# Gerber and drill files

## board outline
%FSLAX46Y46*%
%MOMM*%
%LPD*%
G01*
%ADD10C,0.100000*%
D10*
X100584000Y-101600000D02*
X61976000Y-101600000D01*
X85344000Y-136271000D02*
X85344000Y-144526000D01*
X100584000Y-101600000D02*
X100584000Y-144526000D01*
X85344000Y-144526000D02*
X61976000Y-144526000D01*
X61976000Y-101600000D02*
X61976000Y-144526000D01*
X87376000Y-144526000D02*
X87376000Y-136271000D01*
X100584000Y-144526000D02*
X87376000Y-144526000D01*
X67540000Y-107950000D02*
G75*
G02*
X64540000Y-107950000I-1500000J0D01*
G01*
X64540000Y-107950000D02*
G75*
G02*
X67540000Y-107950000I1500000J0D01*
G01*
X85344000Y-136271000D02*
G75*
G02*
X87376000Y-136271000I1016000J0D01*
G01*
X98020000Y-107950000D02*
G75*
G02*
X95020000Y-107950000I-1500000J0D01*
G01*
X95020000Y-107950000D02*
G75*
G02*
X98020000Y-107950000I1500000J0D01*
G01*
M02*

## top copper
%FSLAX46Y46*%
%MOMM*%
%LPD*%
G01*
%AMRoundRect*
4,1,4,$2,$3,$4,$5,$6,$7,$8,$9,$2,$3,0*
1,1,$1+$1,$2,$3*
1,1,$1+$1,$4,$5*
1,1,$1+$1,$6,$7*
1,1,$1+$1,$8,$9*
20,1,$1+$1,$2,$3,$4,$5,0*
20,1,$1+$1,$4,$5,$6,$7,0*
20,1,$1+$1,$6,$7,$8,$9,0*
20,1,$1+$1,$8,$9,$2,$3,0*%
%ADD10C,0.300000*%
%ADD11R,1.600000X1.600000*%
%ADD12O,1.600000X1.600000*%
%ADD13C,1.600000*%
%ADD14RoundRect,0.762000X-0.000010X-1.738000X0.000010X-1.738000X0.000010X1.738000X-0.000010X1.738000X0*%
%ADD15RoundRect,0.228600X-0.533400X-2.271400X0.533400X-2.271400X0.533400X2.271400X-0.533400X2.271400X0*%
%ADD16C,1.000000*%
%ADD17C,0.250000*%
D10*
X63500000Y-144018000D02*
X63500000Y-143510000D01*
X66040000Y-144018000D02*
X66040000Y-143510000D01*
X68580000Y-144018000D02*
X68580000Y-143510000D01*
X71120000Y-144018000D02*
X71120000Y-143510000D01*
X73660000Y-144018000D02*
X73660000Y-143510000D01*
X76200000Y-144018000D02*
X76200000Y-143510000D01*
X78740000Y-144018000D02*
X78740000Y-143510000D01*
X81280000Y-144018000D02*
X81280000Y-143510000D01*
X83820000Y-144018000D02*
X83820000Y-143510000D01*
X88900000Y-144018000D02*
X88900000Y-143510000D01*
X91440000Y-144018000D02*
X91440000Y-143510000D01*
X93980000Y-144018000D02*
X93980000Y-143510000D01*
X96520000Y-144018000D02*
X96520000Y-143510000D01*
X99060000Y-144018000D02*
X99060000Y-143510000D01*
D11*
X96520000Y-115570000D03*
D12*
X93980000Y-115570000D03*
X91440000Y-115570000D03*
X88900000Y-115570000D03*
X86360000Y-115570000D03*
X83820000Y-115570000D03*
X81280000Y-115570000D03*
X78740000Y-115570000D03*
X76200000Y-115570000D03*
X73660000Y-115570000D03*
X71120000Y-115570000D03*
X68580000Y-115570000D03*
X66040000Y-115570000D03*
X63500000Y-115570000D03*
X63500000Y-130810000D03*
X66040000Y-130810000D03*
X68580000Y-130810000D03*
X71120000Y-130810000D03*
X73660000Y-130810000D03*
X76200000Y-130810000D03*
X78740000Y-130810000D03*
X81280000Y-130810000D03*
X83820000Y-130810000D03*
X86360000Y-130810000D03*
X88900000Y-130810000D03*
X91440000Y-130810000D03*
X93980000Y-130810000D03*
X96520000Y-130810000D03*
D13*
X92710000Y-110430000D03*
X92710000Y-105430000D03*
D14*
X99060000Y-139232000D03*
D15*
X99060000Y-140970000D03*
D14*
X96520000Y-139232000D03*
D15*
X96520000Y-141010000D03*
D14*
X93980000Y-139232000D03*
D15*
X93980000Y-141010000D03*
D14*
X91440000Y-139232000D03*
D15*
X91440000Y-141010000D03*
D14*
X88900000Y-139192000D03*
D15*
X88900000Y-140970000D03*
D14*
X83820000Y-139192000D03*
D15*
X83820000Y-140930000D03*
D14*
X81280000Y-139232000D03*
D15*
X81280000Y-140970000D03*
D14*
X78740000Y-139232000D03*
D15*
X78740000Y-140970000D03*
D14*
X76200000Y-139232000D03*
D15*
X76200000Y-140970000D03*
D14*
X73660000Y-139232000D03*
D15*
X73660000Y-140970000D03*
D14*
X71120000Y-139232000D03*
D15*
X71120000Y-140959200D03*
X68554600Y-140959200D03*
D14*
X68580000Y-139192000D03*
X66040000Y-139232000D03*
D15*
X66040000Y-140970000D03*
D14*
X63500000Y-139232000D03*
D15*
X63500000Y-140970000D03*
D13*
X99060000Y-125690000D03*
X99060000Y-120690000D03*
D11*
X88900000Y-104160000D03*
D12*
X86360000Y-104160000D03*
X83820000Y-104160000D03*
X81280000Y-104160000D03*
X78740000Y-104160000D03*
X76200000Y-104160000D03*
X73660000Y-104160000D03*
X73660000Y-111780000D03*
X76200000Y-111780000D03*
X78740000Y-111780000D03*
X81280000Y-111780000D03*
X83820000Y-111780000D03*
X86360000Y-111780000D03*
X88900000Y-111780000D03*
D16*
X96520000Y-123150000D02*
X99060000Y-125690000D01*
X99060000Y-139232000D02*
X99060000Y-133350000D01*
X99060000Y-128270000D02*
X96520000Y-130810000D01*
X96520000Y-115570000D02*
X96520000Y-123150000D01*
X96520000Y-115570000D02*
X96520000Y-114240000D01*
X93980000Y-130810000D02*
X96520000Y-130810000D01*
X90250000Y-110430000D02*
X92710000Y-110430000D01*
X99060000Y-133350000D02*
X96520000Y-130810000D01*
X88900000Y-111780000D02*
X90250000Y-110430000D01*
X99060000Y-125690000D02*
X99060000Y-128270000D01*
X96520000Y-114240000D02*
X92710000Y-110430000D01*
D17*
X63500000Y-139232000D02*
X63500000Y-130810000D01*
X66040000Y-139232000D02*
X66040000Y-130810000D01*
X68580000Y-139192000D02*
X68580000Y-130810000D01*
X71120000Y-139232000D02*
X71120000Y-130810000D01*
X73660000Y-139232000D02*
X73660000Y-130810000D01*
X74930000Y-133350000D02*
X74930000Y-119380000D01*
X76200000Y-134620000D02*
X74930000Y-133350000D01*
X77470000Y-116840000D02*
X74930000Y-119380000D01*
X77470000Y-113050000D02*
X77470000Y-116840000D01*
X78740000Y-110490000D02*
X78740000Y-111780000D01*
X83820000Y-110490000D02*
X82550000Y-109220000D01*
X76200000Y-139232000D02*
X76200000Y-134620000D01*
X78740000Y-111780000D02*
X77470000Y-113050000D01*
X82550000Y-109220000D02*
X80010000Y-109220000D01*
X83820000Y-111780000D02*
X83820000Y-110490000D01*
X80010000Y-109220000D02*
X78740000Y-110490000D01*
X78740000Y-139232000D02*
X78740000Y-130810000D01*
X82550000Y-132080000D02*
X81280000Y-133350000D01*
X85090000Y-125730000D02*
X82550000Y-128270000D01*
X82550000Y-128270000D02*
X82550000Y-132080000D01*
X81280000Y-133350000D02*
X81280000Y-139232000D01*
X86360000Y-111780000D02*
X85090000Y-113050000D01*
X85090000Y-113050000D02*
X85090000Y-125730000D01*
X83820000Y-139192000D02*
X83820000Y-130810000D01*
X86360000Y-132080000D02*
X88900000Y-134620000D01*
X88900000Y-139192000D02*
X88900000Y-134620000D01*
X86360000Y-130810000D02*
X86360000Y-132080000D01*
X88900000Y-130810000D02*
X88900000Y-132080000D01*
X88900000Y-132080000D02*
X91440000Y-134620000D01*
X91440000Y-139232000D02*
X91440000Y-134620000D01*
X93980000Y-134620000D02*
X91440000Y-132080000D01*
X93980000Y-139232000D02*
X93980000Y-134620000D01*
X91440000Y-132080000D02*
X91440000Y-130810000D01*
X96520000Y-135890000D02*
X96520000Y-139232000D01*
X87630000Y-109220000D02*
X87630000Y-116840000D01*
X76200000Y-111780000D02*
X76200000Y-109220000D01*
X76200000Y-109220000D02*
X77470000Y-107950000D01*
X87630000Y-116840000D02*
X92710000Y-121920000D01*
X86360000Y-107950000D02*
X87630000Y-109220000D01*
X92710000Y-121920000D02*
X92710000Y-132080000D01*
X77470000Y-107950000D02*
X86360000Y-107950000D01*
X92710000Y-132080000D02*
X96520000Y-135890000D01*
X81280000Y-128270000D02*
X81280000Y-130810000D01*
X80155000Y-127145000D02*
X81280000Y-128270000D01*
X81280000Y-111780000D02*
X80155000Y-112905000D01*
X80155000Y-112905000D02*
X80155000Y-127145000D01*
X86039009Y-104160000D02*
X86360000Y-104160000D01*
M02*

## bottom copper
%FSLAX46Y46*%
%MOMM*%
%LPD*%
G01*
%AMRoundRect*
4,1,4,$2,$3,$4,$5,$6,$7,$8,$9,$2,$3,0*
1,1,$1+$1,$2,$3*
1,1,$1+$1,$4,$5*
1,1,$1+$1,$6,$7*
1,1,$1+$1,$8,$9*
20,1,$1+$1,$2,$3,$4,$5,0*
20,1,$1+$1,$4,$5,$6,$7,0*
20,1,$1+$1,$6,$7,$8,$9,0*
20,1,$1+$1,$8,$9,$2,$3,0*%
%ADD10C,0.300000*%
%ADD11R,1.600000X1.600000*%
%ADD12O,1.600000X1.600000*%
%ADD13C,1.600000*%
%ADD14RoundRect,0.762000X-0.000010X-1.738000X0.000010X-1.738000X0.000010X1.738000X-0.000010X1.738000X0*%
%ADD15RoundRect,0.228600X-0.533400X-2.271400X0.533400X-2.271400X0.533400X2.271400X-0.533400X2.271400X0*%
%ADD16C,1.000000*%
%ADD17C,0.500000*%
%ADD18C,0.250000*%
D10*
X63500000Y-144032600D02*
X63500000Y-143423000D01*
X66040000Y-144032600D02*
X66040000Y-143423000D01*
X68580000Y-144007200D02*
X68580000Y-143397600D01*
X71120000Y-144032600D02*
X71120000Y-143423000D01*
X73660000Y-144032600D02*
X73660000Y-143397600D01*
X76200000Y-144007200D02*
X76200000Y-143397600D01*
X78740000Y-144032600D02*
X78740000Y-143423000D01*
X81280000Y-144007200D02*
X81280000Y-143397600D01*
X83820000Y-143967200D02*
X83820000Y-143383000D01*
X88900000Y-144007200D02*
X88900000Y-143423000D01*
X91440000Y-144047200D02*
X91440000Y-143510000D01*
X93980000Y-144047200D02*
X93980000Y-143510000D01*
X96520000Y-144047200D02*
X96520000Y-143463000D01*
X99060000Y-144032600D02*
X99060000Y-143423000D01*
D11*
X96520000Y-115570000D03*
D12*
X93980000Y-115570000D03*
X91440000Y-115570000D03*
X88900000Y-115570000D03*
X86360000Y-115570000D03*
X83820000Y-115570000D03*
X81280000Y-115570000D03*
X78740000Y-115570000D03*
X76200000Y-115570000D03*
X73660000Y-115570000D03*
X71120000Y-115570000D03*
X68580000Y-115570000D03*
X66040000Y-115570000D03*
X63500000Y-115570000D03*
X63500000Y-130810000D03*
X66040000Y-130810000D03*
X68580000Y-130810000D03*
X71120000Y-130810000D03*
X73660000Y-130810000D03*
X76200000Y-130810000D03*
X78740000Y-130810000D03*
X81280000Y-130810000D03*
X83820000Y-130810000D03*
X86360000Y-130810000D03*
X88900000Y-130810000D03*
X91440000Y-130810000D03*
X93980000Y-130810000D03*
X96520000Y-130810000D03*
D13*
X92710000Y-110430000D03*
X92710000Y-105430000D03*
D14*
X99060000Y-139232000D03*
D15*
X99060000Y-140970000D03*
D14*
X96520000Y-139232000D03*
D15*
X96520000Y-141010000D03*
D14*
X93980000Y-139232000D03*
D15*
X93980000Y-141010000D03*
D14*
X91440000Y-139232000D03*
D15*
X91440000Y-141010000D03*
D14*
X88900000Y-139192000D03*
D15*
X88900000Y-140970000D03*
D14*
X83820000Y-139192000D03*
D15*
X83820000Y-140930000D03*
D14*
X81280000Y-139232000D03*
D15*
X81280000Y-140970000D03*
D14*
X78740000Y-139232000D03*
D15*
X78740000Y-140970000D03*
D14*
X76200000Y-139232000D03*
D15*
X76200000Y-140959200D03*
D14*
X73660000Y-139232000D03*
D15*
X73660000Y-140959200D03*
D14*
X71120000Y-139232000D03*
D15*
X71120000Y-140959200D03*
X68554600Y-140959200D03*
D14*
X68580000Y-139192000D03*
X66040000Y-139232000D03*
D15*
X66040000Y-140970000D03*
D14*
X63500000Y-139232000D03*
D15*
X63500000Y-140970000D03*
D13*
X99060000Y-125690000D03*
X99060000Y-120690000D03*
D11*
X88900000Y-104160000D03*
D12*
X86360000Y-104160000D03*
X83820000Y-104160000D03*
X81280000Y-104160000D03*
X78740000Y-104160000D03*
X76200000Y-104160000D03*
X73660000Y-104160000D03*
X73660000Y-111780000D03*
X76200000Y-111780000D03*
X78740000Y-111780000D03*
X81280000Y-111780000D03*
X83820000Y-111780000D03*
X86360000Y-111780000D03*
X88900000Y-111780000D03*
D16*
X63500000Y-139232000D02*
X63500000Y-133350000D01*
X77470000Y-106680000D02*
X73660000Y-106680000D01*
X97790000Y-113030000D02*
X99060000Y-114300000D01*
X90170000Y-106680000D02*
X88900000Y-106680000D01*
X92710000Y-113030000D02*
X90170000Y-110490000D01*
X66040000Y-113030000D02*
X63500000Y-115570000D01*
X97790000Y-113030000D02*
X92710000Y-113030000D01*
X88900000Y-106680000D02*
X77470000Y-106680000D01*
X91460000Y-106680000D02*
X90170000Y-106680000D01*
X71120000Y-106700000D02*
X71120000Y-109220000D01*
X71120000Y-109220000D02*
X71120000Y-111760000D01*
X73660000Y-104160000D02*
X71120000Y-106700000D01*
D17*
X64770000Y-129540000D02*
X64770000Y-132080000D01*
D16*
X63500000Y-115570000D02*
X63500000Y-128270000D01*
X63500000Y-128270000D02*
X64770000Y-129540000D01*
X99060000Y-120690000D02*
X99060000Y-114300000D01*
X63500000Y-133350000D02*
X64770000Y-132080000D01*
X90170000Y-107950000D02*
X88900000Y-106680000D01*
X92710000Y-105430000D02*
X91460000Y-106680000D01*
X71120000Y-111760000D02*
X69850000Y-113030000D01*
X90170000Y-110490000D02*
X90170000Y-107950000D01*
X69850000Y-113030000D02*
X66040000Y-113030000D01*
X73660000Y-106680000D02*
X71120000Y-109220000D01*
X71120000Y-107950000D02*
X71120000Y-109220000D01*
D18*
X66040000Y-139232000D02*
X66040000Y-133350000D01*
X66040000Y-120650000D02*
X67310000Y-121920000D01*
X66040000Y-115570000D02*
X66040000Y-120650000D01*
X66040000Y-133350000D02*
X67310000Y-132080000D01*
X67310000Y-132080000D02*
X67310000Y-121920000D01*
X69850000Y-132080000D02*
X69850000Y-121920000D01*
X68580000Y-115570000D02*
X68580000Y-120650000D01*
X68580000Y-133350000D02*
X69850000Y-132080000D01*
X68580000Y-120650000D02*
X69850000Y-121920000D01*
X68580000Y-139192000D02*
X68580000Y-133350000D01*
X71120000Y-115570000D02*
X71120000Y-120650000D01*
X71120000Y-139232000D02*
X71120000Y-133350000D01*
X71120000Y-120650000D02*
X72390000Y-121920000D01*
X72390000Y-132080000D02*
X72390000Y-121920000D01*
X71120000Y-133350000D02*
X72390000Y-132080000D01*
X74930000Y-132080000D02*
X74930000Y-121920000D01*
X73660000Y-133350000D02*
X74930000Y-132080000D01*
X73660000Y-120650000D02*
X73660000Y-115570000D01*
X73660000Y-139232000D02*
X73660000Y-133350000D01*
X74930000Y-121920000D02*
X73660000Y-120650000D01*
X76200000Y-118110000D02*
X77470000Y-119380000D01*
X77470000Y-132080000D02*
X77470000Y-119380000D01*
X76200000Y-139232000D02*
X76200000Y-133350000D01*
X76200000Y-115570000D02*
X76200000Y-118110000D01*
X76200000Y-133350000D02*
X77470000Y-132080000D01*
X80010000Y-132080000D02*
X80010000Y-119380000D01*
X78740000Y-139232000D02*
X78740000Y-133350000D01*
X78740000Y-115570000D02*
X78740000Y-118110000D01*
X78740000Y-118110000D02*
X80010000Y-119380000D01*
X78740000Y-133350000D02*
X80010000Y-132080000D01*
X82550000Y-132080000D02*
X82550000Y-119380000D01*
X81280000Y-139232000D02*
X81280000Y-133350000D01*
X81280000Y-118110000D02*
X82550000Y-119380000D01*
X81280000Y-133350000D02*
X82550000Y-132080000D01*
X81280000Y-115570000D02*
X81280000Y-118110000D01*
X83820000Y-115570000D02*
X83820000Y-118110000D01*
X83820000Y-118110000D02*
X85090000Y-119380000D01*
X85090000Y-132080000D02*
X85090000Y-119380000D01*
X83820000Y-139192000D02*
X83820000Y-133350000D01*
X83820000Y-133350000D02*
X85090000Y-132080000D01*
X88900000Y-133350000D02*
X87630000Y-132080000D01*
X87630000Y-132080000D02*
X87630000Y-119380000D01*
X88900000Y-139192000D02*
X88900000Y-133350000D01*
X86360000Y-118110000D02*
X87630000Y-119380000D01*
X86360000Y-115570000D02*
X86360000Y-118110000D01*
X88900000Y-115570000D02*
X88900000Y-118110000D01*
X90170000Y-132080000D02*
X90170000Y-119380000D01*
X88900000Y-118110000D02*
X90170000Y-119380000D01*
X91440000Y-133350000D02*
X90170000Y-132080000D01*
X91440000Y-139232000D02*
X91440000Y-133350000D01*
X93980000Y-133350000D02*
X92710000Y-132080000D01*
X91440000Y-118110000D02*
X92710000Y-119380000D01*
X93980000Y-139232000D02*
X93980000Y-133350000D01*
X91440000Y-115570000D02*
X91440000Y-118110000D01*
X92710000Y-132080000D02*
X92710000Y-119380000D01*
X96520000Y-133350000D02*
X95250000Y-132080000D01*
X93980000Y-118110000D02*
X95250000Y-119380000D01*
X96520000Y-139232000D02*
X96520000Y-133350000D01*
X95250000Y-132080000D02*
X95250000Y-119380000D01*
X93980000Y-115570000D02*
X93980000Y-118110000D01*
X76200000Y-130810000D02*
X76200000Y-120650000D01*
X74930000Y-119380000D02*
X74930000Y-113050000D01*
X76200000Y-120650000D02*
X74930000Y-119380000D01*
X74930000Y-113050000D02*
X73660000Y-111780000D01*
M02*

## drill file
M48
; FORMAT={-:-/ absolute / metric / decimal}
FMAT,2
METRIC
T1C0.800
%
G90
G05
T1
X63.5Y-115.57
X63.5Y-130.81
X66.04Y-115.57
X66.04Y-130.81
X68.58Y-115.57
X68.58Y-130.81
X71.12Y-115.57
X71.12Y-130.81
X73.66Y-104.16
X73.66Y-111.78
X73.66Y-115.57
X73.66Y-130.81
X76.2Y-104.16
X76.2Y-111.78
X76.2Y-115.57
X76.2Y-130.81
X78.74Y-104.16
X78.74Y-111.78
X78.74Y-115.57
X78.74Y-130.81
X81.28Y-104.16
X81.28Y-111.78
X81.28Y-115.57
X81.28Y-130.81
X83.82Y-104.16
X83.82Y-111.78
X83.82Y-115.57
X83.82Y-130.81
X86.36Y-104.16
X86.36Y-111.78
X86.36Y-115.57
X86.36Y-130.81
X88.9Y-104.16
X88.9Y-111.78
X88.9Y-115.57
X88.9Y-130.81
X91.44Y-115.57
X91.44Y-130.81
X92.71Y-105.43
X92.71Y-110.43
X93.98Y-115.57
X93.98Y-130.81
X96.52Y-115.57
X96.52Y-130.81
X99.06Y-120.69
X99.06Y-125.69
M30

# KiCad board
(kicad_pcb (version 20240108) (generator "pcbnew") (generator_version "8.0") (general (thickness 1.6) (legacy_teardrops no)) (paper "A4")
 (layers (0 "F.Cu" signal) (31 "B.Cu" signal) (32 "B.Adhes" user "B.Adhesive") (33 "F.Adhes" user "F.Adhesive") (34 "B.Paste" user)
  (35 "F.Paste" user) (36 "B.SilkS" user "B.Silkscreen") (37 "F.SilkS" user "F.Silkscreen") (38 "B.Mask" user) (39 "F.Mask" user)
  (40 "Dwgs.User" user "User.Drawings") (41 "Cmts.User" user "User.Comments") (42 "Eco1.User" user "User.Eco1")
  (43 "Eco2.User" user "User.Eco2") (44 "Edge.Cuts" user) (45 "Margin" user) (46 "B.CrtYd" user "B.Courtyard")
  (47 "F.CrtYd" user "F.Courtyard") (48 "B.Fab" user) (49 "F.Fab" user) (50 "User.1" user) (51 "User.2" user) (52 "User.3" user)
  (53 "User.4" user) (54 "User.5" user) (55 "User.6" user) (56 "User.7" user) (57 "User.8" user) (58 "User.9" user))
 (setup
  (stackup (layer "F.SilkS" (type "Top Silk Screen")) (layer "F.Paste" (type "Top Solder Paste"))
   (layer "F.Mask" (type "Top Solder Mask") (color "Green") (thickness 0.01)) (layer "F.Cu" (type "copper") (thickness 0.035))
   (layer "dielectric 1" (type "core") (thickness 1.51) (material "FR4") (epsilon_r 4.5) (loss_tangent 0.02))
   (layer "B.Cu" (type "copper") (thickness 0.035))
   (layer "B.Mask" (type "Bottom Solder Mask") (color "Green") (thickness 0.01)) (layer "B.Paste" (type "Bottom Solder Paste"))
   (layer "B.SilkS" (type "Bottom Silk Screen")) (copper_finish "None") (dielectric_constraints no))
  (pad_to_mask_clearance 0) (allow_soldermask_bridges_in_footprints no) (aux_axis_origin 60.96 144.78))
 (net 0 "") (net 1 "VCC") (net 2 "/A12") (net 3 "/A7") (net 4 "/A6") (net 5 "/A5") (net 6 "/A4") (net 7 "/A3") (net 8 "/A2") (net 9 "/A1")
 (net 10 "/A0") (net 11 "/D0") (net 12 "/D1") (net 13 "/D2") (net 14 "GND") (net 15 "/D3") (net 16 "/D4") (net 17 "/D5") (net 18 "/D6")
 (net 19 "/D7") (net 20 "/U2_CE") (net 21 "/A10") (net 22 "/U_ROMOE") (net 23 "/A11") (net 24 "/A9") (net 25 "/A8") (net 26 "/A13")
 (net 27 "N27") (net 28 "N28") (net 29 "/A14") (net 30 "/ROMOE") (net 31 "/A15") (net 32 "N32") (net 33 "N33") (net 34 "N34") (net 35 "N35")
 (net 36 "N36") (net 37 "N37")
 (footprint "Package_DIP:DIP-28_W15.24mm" (layer "F.Cu") (at 96.52 115.57 -90)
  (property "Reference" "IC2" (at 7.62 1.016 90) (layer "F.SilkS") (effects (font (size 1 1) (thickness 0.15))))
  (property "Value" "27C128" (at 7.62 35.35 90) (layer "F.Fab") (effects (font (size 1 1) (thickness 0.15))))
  (pad "1" thru_hole rect (at 0 0 270) (size 1.6 1.6) (drill 0.8) (layers "*.Cu" "*.Mask") (remove_unused_layers no) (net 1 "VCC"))
  (pad "2" thru_hole oval (at 0 2.54 270) (size 1.6 1.6) (drill 0.8) (layers "*.Cu" "*.Mask") (remove_unused_layers no) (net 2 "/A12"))
  (pad "3" thru_hole oval (at 0 5.08 270) (size 1.6 1.6) (drill 0.8) (layers "*.Cu" "*.Mask") (remove_unused_layers no) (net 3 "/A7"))
  (pad "4" thru_hole oval (at 0 7.62 270) (size 1.6 1.6) (drill 0.8) (layers "*.Cu" "*.Mask") (remove_unused_layers no) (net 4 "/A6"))
  (pad "5" thru_hole oval (at 0 10.16 270) (size 1.6 1.6) (drill 0.8) (layers "*.Cu" "*.Mask") (remove_unused_layers no) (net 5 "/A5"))
  (pad "6" thru_hole oval (at 0 12.7 270) (size 1.6 1.6) (drill 0.8) (layers "*.Cu" "*.Mask") (remove_unused_layers no) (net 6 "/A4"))
  (pad "7" thru_hole oval (at 0 15.24 270) (size 1.6 1.6) (drill 0.8) (layers "*.Cu" "*.Mask") (remove_unused_layers no) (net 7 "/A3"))
  (pad "8" thru_hole oval (at 0 17.78 270) (size 1.6 1.6) (drill 0.8) (layers "*.Cu" "*.Mask") (remove_unused_layers no) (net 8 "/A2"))
  (pad "9" thru_hole oval (at 0 20.32 270) (size 1.6 1.6) (drill 0.8) (layers "*.Cu" "*.Mask") (remove_unused_layers no) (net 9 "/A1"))
  (pad "10" thru_hole oval (at 0 22.86 270) (size 1.6 1.6) (drill 0.8) (layers "*.Cu" "*.Mask") (remove_unused_layers no) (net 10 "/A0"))
  (pad "11" thru_hole oval (at 0 25.4 270) (size 1.6 1.6) (drill 0.8) (layers "*.Cu" "*.Mask") (remove_unused_layers no) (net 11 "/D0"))
  (pad "12" thru_hole oval (at 0 27.94 270) (size 1.6 1.6) (drill 0.8) (layers "*.Cu" "*.Mask") (remove_unused_layers no) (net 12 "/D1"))
  (pad "13" thru_hole oval (at 0 30.48 270) (size 1.6 1.6) (drill 0.8) (layers "*.Cu" "*.Mask") (remove_unused_layers no) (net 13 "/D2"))
  (pad "14" thru_hole oval (at 0 33.02 270) (size 1.6 1.6) (drill 0.8) (layers "*.Cu" "*.Mask") (remove_unused_layers no) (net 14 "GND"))
  (pad "15" thru_hole oval (at 15.24 33.02 270) (size 1.6 1.6) (drill 0.8) (layers "*.Cu" "*.Mask") (remove_unused_layers no) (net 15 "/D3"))
  (pad "16" thru_hole oval (at 15.24 30.48 270) (size 1.6 1.6) (drill 0.8) (layers "*.Cu" "*.Mask") (remove_unused_layers no) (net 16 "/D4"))
  (pad "17" thru_hole oval (at 15.24 27.94 270) (size 1.6 1.6) (drill 0.8) (layers "*.Cu" "*.Mask") (remove_unused_layers no) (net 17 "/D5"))
  (pad "18" thru_hole oval (at 15.24 25.4 270) (size 1.6 1.6) (drill 0.8) (layers "*.Cu" "*.Mask") (remove_unused_layers no) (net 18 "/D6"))
  (pad "19" thru_hole oval (at 15.24 22.86 270) (size 1.6 1.6) (drill 0.8) (layers "*.Cu" "*.Mask") (remove_unused_layers no) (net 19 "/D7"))
  (pad "20" thru_hole oval (at 15.24 20.32 270) (size 1.6 1.6) (drill 0.8) (layers "*.Cu" "*.Mask") (remove_unused_layers no)
   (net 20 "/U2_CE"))
  (pad "21" thru_hole oval (at 15.24 17.78 270) (size 1.6 1.6) (drill 0.8) (layers "*.Cu" "*.Mask") (remove_unused_layers no)
   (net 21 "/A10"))
  (pad "22" thru_hole oval (at 15.24 15.24 270) (size 1.6 1.6) (drill 0.8) (layers "*.Cu" "*.Mask") (remove_unused_layers no)
   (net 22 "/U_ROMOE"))
  (pad "23" thru_hole oval (at 15.24 12.7 270) (size 1.6 1.6) (drill 0.8) (layers "*.Cu" "*.Mask") (remove_unused_layers no) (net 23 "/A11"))
  (pad "24" thru_hole oval (at 15.24 10.16 270) (size 1.6 1.6) (drill 0.8) (layers "*.Cu" "*.Mask") (remove_unused_layers no) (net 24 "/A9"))
  (pad "25" thru_hole oval (at 15.24 7.62 270) (size 1.6 1.6) (drill 0.8) (layers "*.Cu" "*.Mask") (remove_unused_layers no) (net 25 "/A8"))
  (pad "26" thru_hole oval (at 15.24 5.08 270) (size 1.6 1.6) (drill 0.8) (layers "*.Cu" "*.Mask") (remove_unused_layers no) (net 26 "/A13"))
  (pad "27" thru_hole oval (at 15.24 2.54 270) (size 1.6 1.6) (drill 0.8) (layers "*.Cu" "*.Mask") (remove_unused_layers no) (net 1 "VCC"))
  (pad "28" thru_hole oval (at 15.24 0 270) (size 1.6 1.6) (drill 0.8) (layers "*.Cu" "*.Mask") (remove_unused_layers no) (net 1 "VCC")))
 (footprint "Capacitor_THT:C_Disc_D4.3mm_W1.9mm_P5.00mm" (layer "F.Cu") (at 92.71 110.43 90)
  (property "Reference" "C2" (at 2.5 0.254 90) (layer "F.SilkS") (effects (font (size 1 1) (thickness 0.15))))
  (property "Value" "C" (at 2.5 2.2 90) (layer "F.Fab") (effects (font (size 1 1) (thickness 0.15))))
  (pad "1" thru_hole circle (at 0 0 90) (size 1.6 1.6) (drill 0.8) (layers "*.Cu" "*.Mask") (remove_unused_layers no) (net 1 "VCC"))
  (pad "2" thru_hole circle (at 5 0 90) (size 1.6 1.6) (drill 0.8) (layers "*.Cu" "*.Mask") (remove_unused_layers no) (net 14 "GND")))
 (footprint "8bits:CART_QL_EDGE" (layer "F.Cu") (at 73.66 139.994)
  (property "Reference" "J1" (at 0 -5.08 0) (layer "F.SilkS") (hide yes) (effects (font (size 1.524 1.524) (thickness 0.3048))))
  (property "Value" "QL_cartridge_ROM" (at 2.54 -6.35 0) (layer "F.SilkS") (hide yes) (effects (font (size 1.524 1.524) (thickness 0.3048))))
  (fp_line (start -10.16 4.024) (end -10.16 3.516) (stroke (width 0.3) (type solid)) (layer "F.Cu"))
  (fp_line (start -7.62 4.024) (end -7.62 3.516) (stroke (width 0.3) (type solid)) (layer "F.Cu"))
  (fp_line (start -5.08 4.024) (end -5.08 3.516) (stroke (width 0.3) (type solid)) (layer "F.Cu"))
  (fp_line (start -2.54 4.024) (end -2.54 3.516) (stroke (width 0.3) (type solid)) (layer "F.Cu"))
  (fp_line (start 0 4.024) (end 0 3.516) (stroke (width 0.3) (type solid)) (layer "F.Cu"))
  (fp_line (start 2.54 4.024) (end 2.54 3.516) (stroke (width 0.3) (type solid)) (layer "F.Cu"))
  (fp_line (start 5.08 4.024) (end 5.08 3.516) (stroke (width 0.3) (type solid)) (layer "F.Cu"))
  (fp_line (start 7.62 4.024) (end 7.62 3.516) (stroke (width 0.3) (type solid)) (layer "F.Cu"))
  (fp_line (start 10.16 4.024) (end 10.16 3.516) (stroke (width 0.3) (type solid)) (layer "F.Cu"))
  (fp_line (start 15.24 4.024) (end 15.24 3.516) (stroke (width 0.3) (type solid)) (layer "F.Cu"))
  (fp_line (start 17.78 4.024) (end 17.78 3.516) (stroke (width 0.3) (type solid)) (layer "F.Cu"))
  (fp_line (start 20.32 4.024) (end 20.32 3.516) (stroke (width 0.3) (type solid)) (layer "F.Cu"))
  (fp_line (start 22.86 4.024) (end 22.86 3.516) (stroke (width 0.3) (type solid)) (layer "F.Cu"))
  (fp_line (start 25.4 4.024) (end 25.4 3.516) (stroke (width 0.3) (type solid)) (layer "F.Cu"))
  (fp_line (start -10.16 4.0386) (end -10.16 3.429) (stroke (width 0.3) (type solid)) (layer "B.Cu"))
  (fp_line (start -7.62 4.0386) (end -7.62 3.429) (stroke (width 0.3) (type solid)) (layer "B.Cu"))
  (fp_line (start -5.08 4.0132) (end -5.08 3.4036) (stroke (width 0.3) (type solid)) (layer "B.Cu"))
  (fp_line (start -2.54 4.0386) (end -2.54 3.429) (stroke (width 0.3) (type solid)) (layer "B.Cu"))
  (fp_line (start 0 4.0386) (end 0 3.4036) (stroke (width 0.3) (type solid)) (layer "B.Cu"))
  (fp_line (start 2.54 4.0132) (end 2.54 3.4036) (stroke (width 0.3) (type solid)) (layer "B.Cu"))
  (fp_line (start 5.08 4.0386) (end 5.08 3.429) (stroke (width 0.3) (type solid)) (layer "B.Cu"))
  (fp_line (start 7.62 4.0132) (end 7.62 3.4036) (stroke (width 0.3) (type solid)) (layer "B.Cu"))
  (fp_line (start 10.16 3.9732) (end 10.16 3.389) (stroke (width 0.3) (type solid)) (layer "B.Cu"))
  (fp_line (start 15.24 4.0132) (end 15.24 3.429) (stroke (width 0.3) (type solid)) (layer "B.Cu"))
  (fp_line (start 17.78 4.0532) (end 17.78 3.516) (stroke (width 0.3) (type solid)) (layer "B.Cu"))
  (fp_line (start 20.32 4.0532) (end 20.32 3.516) (stroke (width 0.3) (type solid)) (layer "B.Cu"))
  (fp_line (start 22.86 4.0532) (end 22.86 3.469) (stroke (width 0.3) (type solid)) (layer "B.Cu"))
  (fp_line (start 25.4 4.0386) (end 25.4 3.429) (stroke (width 0.3) (type solid)) (layer "B.Cu"))
  (pad "1" connect roundrect (at 25.4 -0.762) (size 1.524 5) (layers "F.Cu") (roundrect_rratio 0.5) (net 1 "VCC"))
  (pad "1" connect roundrect (at 25.4 0.976) (size 1.524 5) (layers "F.Cu") (roundrect_rratio 0.15) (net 1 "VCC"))
  (pad "2" connect roundrect (at 25.4 -0.762) (size 1.524 5) (layers "B.Cu") (roundrect_rratio 0.5) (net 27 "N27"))
  (pad "2" connect roundrect (at 25.4 0.976) (size 1.524 5) (layers "B.Cu") (roundrect_rratio 0.15) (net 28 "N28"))
  (pad "3" connect roundrect (at 22.86 -0.762) (size 1.524 5) (layers "F.Cu") (roundrect_rratio 0.5) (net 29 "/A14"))
  (pad "3" connect roundrect (at 22.86 1.016) (size 1.524 5) (layers "F.Cu") (roundrect_rratio 0.15) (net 29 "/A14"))
  (pad "4" connect roundrect (at 22.86 -0.762) (size 1.524 5) (layers "B.Cu") (roundrect_rratio 0.5) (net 2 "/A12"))
  (pad "4" connect roundrect (at 22.86 1.016) (size 1.524 5) (layers "B.Cu") (roundrect_rratio 0.15) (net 2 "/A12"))
  (pad "5" connect roundrect (at 20.32 -0.762) (size 1.524 5) (layers "F.Cu") (roundrect_rratio 0.5) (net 26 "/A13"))
  (pad "5" connect roundrect (at 20.32 1.016) (size 1.524 5) (layers "F.Cu") (roundrect_rratio 0.15) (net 26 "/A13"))
  (pad "6" connect roundrect (at 20.32 -0.762) (size 1.524 5) (layers "B.Cu") (roundrect_rratio 0.5) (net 3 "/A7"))
  (pad "6" connect roundrect (at 20.32 1.016) (size 1.524 5) (layers "B.Cu") (roundrect_rratio 0.15) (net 3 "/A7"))
  (pad "7" connect roundrect (at 17.78 -0.762) (size 1.524 5) (layers "F.Cu") (roundrect_rratio 0.5) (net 25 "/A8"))
  (pad "7" connect roundrect (at 17.78 1.016) (size 1.524 5) (layers "F.Cu") (roundrect_rratio 0.15) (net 25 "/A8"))
  (pad "8" connect roundrect (at 17.78 -0.762) (size 1.524 5) (layers "B.Cu") (roundrect_rratio 0.5) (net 4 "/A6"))
  (pad "8" connect roundrect (at 17.78 1.016) (size 1.524 5) (layers "B.Cu") (roundrect_rratio 0.15) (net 4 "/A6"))
  (pad "9" connect roundrect (at 15.24 -0.802) (size 1.524 5) (layers "F.Cu") (roundrect_rratio 0.5) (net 24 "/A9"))
  (pad "9" connect roundrect (at 15.24 0.976) (size 1.524 5) (layers "F.Cu") (roundrect_rratio 0.15) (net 24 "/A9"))
  (pad "10" connect roundrect (at 15.24 -0.802) (size 1.524 5) (layers "B.Cu") (roundrect_rratio 0.5) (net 5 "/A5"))
  (pad "10" connect roundrect (at 15.24 0.976) (size 1.524 5) (layers "B.Cu") (roundrect_rratio 0.15) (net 5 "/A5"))
  (pad "11" connect roundrect (at 10.16 -0.802) (size 1.524 5) (layers "F.Cu") (roundrect_rratio 0.5) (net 23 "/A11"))
  (pad "11" connect roundrect (at 10.16 0.936) (size 1.524 5) (layers "F.Cu") (roundrect_rratio 0.15) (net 23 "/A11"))
  (pad "12" connect roundrect (at 10.16 -0.802) (size 1.524 5) (layers "B.Cu") (roundrect_rratio 0.5) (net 6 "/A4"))
  (pad "12" connect roundrect (at 10.16 0.936) (size 1.524 5) (layers "B.Cu") (roundrect_rratio 0.15) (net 6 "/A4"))
  (pad "13" connect roundrect (at 7.62 -0.762) (size 1.524 5) (layers "F.Cu") (roundrect_rratio 0.5) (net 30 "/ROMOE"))
  (pad "13" connect roundrect (at 7.62 0.976) (size 1.524 5) (layers "F.Cu") (roundrect_rratio 0.15) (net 30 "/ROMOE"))
  (pad "14" connect roundrect (at 7.62 -0.762) (size 1.524 5) (layers "B.Cu") (roundrect_rratio 0.5) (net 7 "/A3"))
  (pad "14" connect roundrect (at 7.62 0.976) (size 1.524 5) (layers "B.Cu") (roundrect_rratio 0.15) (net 7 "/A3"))
  (pad "15" connect roundrect (at 5.08 -0.762) (size 1.524 5) (layers "F.Cu") (roundrect_rratio 0.5) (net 21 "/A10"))
  (pad "15" connect roundrect (at 5.08 0.976) (size 1.524 5) (layers "F.Cu") (roundrect_rratio 0.15) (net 21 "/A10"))
  (pad "16" connect roundrect (at 5.08 -0.762) (size 1.524 5) (layers "B.Cu") (roundrect_rratio 0.5) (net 8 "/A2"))
  (pad "16" connect roundrect (at 5.08 0.976) (size 1.524 5) (layers "B.Cu") (roundrect_rratio 0.15) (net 8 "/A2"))
  (pad "17" connect roundrect (at 2.54 -0.762) (size 1.524 5) (layers "F.Cu") (roundrect_rratio 0.5) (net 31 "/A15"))
  (pad "17" connect roundrect (at 2.54 0.976) (size 1.524 5) (layers "F.Cu") (roundrect_rratio 0.15) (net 31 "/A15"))
  (pad "18" connect roundrect (at 2.54 -0.762) (size 1.524 5) (layers "B.Cu") (roundrect_rratio 0.5) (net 9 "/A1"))
  (pad "18" connect roundrect (at 2.54 0.9652) (size 1.524 5) (layers "B.Cu") (roundrect_rratio 0.15) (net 9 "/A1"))
  (pad "19" connect roundrect (at 0 -0.762) (size 1.524 5) (layers "F.Cu") (roundrect_rratio 0.5) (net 19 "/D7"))
  (pad "19" connect roundrect (at 0 0.976) (size 1.524 5) (layers "F.Cu") (roundrect_rratio 0.15) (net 19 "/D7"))
  (pad "20" connect roundrect (at 0 -0.762) (size 1.524 5) (layers "B.Cu") (roundrect_rratio 0.5) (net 10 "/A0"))
  (pad "20" connect roundrect (at 0 0.9652) (size 1.524 5) (layers "B.Cu") (roundrect_rratio 0.15) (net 10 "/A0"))
  (pad "21" connect roundrect (at -2.54 -0.762) (size 1.524 5) (layers "F.Cu") (roundrect_rratio 0.5) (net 18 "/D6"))
  (pad "21" connect roundrect (at -2.54 0.9652) (size 1.524 5) (layers "F.Cu") (roundrect_rratio 0.15) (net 18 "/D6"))
  (pad "22" connect roundrect (at -2.54 -0.762) (size 1.524 5) (layers "B.Cu") (roundrect_rratio 0.5) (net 11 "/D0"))
  (pad "22" connect roundrect (at -2.54 0.9652) (size 1.524 5) (layers "B.Cu") (roundrect_rratio 0.15) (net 11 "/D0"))
  (pad "23" connect roundrect (at -5.1054 0.9652) (size 1.524 5) (layers "F.Cu") (roundrect_rratio 0.15) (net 17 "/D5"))
  (pad "23" connect roundrect (at -5.08 -0.802) (size 1.524 5) (layers "F.Cu") (roundrect_rratio 0.5) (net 17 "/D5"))
  (pad "24" connect roundrect (at -5.1054 0.9652) (size 1.524 5) (layers "B.Cu") (roundrect_rratio 0.15) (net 12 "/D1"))
  (pad "24" connect roundrect (at -5.08 -0.802) (size 1.524 5) (layers "B.Cu") (roundrect_rratio 0.5) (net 12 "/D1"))
  (pad "25" connect roundrect (at -7.62 -0.762) (size 1.524 5) (layers "F.Cu") (roundrect_rratio 0.5) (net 16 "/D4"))
  (pad "25" connect roundrect (at -7.62 0.976) (size 1.524 5) (layers "F.Cu") (roundrect_rratio 0.15) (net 16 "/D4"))
  (pad "26" connect roundrect (at -7.62 -0.762) (size 1.524 5) (layers "B.Cu") (roundrect_rratio 0.5) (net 13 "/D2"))
  (pad "26" connect roundrect (at -7.62 0.976) (size 1.524 5) (layers "B.Cu") (roundrect_rratio 0.15) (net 13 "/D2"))
  (pad "27" connect roundrect (at -10.16 -0.762) (size 1.524 5) (layers "F.Cu") (roundrect_rratio 0.5) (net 15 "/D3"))
  (pad "27" connect roundrect (at -10.16 0.976) (size 1.524 5) (layers "F.Cu") (roundrect_rratio 0.15) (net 15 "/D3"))
  (pad "28" connect roundrect (at -10.16 -0.762) (size 1.524 5) (layers "B.Cu") (roundrect_rratio 0.5) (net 14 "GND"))
  (pad "28" connect roundrect (at -10.16 0.976) (size 1.524 5) (layers "B.Cu") (roundrect_rratio 0.15) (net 14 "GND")))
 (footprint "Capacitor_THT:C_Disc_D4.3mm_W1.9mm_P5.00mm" (layer "F.Cu") (at 99.06 125.69 90)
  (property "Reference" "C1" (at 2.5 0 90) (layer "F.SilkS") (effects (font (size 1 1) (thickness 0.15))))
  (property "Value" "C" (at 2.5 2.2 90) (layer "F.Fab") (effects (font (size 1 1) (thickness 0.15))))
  (pad "1" thru_hole circle (at 0 0 90) (size 1.6 1.6) (drill 0.8) (layers "*.Cu" "*.Mask") (remove_unused_layers no) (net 1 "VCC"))
  (pad "2" thru_hole circle (at 5 0 90) (size 1.6 1.6) (drill 0.8) (layers "*.Cu" "*.Mask") (remove_unused_layers no) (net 14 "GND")))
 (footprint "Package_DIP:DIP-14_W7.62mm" (layer "F.Cu") (at 88.9 104.16 -90)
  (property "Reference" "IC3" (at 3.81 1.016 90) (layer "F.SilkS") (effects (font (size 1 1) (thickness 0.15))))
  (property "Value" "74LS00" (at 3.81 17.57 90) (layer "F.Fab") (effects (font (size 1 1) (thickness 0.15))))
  (pad "1" thru_hole rect (at 0 0 270) (size 1.6 1.6) (drill 0.8) (layers "*.Cu" "*.Mask") (remove_unused_layers no) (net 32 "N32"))
  (pad "2" thru_hole oval (at 0 2.54 270) (size 1.6 1.6) (drill 0.8) (layers "*.Cu" "*.Mask") (remove_unused_layers no) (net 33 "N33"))
  (pad "3" thru_hole oval (at 0 5.08 270) (size 1.6 1.6) (drill 0.8) (layers "*.Cu" "*.Mask") (remove_unused_layers no) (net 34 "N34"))
  (pad "4" thru_hole oval (at 0 7.62 270) (size 1.6 1.6) (drill 0.8) (layers "*.Cu" "*.Mask") (remove_unused_layers no) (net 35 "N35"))
  (pad "5" thru_hole oval (at 0 10.16 270) (size 1.6 1.6) (drill 0.8) (layers "*.Cu" "*.Mask") (remove_unused_layers no) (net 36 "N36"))
  (pad "6" thru_hole oval (at 0 12.7 270) (size 1.6 1.6) (drill 0.8) (layers "*.Cu" "*.Mask") (remove_unused_layers no) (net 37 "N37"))
  (pad "7" thru_hole oval (at 0 15.24 270) (size 1.6 1.6) (drill 0.8) (layers "*.Cu" "*.Mask") (remove_unused_layers no) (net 14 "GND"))
  (pad "8" thru_hole oval (at 7.62 15.24 270) (size 1.6 1.6) (drill 0.8) (layers "*.Cu" "*.Mask") (remove_unused_layers no)
   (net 20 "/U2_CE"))
  (pad "9" thru_hole oval (at 7.62 12.7 270) (size 1.6 1.6) (drill 0.8) (layers "*.Cu" "*.Mask") (remove_unused_layers no) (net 29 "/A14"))
  (pad "10" thru_hole oval (at 7.62 10.16 270) (size 1.6 1.6) (drill 0.8) (layers "*.Cu" "*.Mask") (remove_unused_layers no) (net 31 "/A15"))
  (pad "11" thru_hole oval (at 7.62 7.62 270) (size 1.6 1.6) (drill 0.8) (layers "*.Cu" "*.Mask") (remove_unused_layers no)
   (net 22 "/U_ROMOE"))
  (pad "12" thru_hole oval (at 7.62 5.08 270) (size 1.6 1.6) (drill 0.8) (layers "*.Cu" "*.Mask") (remove_unused_layers no) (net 31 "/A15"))
  (pad "13" thru_hole oval (at 7.62 2.54 270) (size 1.6 1.6) (drill 0.8) (layers "*.Cu" "*.Mask") (remove_unused_layers no)
   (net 30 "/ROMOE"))
  (pad "14" thru_hole oval (at 7.62 0 270) (size 1.6 1.6) (drill 0.8) (layers "*.Cu" "*.Mask") (remove_unused_layers no) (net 1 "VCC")))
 (gr_line (start 100.584 101.6) (end 61.976 101.6) (stroke (width 0.1) (type solid)) (layer "Edge.Cuts"))
 (gr_line (start 85.344 136.271) (end 85.344 144.526) (stroke (width 0.1) (type solid)) (layer "Edge.Cuts"))
 (gr_line (start 100.584 101.6) (end 100.584 144.526) (stroke (width 0.1) (type solid)) (layer "Edge.Cuts"))
 (gr_line (start 85.344 144.526) (end 61.976 144.526) (stroke (width 0.1) (type solid)) (layer "Edge.Cuts"))
 (gr_line (start 61.976 101.6) (end 61.976 144.526) (stroke (width 0.1) (type solid)) (layer "Edge.Cuts"))
 (gr_line (start 87.376 144.526) (end 87.376 136.271) (stroke (width 0.1) (type solid)) (layer "Edge.Cuts"))
 (gr_line (start 100.584 144.526) (end 87.376 144.526) (stroke (width 0.1) (type solid)) (layer "Edge.Cuts"))
 (gr_circle (center 66.04 107.95) (end 67.54 107.95) (stroke (width 0.1) (type default)) (fill none) (layer "Edge.Cuts"))
 (gr_arc (start 85.344 136.271) (mid 86.36 135.255) (end 87.376 136.271) (stroke (width 0.1) (type solid)) (layer "Edge.Cuts"))
 (gr_circle (center 96.52 107.95) (end 98.02 107.95) (stroke (width 0.1) (type default)) (fill none) (layer "Edge.Cuts"))
 (segment (start 96.52 123.15) (end 99.06 125.69) (width 1) (layer "F.Cu") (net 1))
 (segment (start 99.06 139.232) (end 99.06 133.35) (width 1) (layer "F.Cu") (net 1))
 (segment (start 99.06 128.27) (end 96.52 130.81) (width 1) (layer "F.Cu") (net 1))
 (segment (start 96.52 115.57) (end 96.52 123.15) (width 1) (layer "F.Cu") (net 1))
 (segment (start 96.52 115.57) (end 96.52 114.24) (width 1) (layer "F.Cu") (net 1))
 (segment (start 93.98 130.81) (end 96.52 130.81) (width 1) (layer "F.Cu") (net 1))
 (segment (start 90.25 110.43) (end 92.71 110.43) (width 1) (layer "F.Cu") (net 1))
 (segment (start 99.06 133.35) (end 96.52 130.81) (width 1) (layer "F.Cu") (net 1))
 (segment (start 88.9 111.78) (end 90.25 110.43) (width 1) (layer "F.Cu") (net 1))
 (segment (start 99.06 125.69) (end 99.06 128.27) (width 1) (layer "F.Cu") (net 1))
 (segment (start 96.52 114.24) (end 92.71 110.43) (width 1) (layer "F.Cu") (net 1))
 (segment (start 63.5 139.232) (end 63.5 133.35) (width 1) (layer "B.Cu") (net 14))
 (segment (start 77.47 106.68) (end 73.66 106.68) (width 1) (layer "B.Cu") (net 14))
 (segment (start 97.79 113.03) (end 99.06 114.3) (width 1) (layer "B.Cu") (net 14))
 (segment (start 90.17 106.68) (end 88.9 106.68) (width 1) (layer "B.Cu") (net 14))
 (segment (start 92.71 113.03) (end 90.17 110.49) (width 1) (layer "B.Cu") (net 14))
 (segment (start 66.04 113.03) (end 63.5 115.57) (width 1) (layer "B.Cu") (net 14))
 (segment (start 97.79 113.03) (end 92.71 113.03) (width 1) (layer "B.Cu") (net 14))
 (segment (start 88.9 106.68) (end 77.47 106.68) (width 1) (layer "B.Cu") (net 14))
 (segment (start 91.46 106.68) (end 90.17 106.68) (width 1) (layer "B.Cu") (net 14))
 (segment (start 71.12 106.7) (end 71.12 109.22) (width 1) (layer "B.Cu") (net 14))
 (segment (start 71.12 109.22) (end 71.12 111.76) (width 1) (layer "B.Cu") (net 14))
 (segment (start 73.66 104.16) (end 71.12 106.7) (width 1) (layer "B.Cu") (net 14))
 (segment (start 64.77 129.54) (end 64.77 132.08) (width 0.5) (layer "B.Cu") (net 14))
 (segment (start 63.5 115.57) (end 63.5 128.27) (width 1) (layer "B.Cu") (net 14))
 (segment (start 63.5 128.27) (end 64.77 129.54) (width 1) (layer "B.Cu") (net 14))
 (segment (start 99.06 120.69) (end 99.06 114.3) (width 1) (layer "B.Cu") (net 14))
 (segment (start 63.5 133.35) (end 64.77 132.08) (width 1) (layer "B.Cu") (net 14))
 (segment (start 90.17 107.95) (end 88.9 106.68) (width 1) (layer "B.Cu") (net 14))
 (segment (start 92.71 105.43) (end 91.46 106.68) (width 1) (layer "B.Cu") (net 14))
 (segment (start 71.12 111.76) (end 69.85 113.03) (width 1) (layer "B.Cu") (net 14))
 (segment (start 90.17 110.49) (end 90.17 107.95) (width 1) (layer "B.Cu") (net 14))
 (segment (start 69.85 113.03) (end 66.04 113.03) (width 1) (layer "B.Cu") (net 14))
 (segment (start 73.66 106.68) (end 71.12 109.22) (width 1) (layer "B.Cu") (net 14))
 (segment (start 71.12 107.95) (end 71.12 109.22) (width 1) (layer "B.Cu") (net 14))
 (segment (start 63.5 139.232) (end 63.5 130.81) (width 0.25) (layer "F.Cu") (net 15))
 (segment (start 66.04 139.232) (end 66.04 130.81) (width 0.25) (layer "F.Cu") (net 16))
 (segment (start 66.04 139.232) (end 66.04 133.35) (width 0.25) (layer "B.Cu") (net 13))
 (segment (start 66.04 120.65) (end 67.31 121.92) (width 0.25) (layer "B.Cu") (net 13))
 (segment (start 66.04 115.57) (end 66.04 120.65) (width 0.25) (layer "B.Cu") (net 13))
 (segment (start 66.04 133.35) (end 67.31 132.08) (width 0.25) (layer "B.Cu") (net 13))
 (segment (start 67.31 132.08) (end 67.31 121.92) (width 0.25) (layer "B.Cu") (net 13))
 (segment (start 68.58 139.192) (end 68.58 130.81) (width 0.25) (layer "F.Cu") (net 17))
 (segment (start 69.85 132.08) (end 69.85 121.92) (width 0.25) (layer "B.Cu") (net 12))
 (segment (start 68.58 115.57) (end 68.58 120.65) (width 0.25) (layer "B.Cu") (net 12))
 (segment (start 68.58 133.35) (end 69.85 132.08) (width 0.25) (layer "B.Cu") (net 12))
 (segment (start 68.58 120.65) (end 69.85 121.92) (width 0.25) (layer "B.Cu") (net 12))
 (segment (start 68.58 139.192) (end 68.58 133.35) (width 0.25) (layer "B.Cu") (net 12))
 (segment (start 71.12 139.232) (end 71.12 130.81) (width 0.25) (layer "F.Cu") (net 18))
 (segment (start 71.12 115.57) (end 71.12 120.65) (width 0.25) (layer "B.Cu") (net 11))
 (segment (start 71.12 139.232) (end 71.12 133.35) (width 0.25) (layer "B.Cu") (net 11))
 (segment (start 71.12 120.65) (end 72.39 121.92) (width 0.25) (layer "B.Cu") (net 11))
 (segment (start 72.39 132.08) (end 72.39 121.92) (width 0.25) (layer "B.Cu") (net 11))
 (segment (start 71.12 133.35) (end 72.39 132.08) (width 0.25) (layer "B.Cu") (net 11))
 (segment (start 73.66 139.232) (end 73.66 130.81) (width 0.25) (layer "F.Cu") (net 19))
 (segment (start 74.93 132.08) (end 74.93 121.92) (width 0.25) (layer "B.Cu") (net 10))
 (segment (start 73.66 133.35) (end 74.93 132.08) (width 0.25) (layer "B.Cu") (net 10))
 (segment (start 73.66 120.65) (end 73.66 115.57) (width 0.25) (layer "B.Cu") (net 10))
 (segment (start 73.66 139.232) (end 73.66 133.35) (width 0.25) (layer "B.Cu") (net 10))
 (segment (start 74.93 121.92) (end 73.66 120.65) (width 0.25) (layer "B.Cu") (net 10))
 (segment (start 74.93 133.35) (end 74.93 119.38) (width 0.25) (layer "F.Cu") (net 31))
 (segment (start 76.2 134.62) (end 74.93 133.35) (width 0.25) (layer "F.Cu") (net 31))
 (segment (start 77.47 116.84) (end 74.93 119.38) (width 0.25) (layer "F.Cu") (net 31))
 (segment (start 77.47 113.05) (end 77.47 116.84) (width 0.25) (layer "F.Cu") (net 31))
 (segment (start 78.74 110.49) (end 78.74 111.78) (width 0.25) (layer "F.Cu") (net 31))
 (segment (start 83.82 110.49) (end 82.55 109.22) (width 0.25) (layer "F.Cu") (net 31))
 (segment (start 76.2 139.232) (end 76.2 134.62) (width 0.25) (layer "F.Cu") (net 31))
 (segment (start 78.74 111.78) (end 77.47 113.05) (width 0.25) (layer "F.Cu") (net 31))
 (segment (start 82.55 109.22) (end 80.01 109.22) (width 0.25) (layer "F.Cu") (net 31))
 (segment (start 83.82 111.78) (end 83.82 110.49) (width 0.25) (layer "F.Cu") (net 31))
 (segment (start 80.01 109.22) (end 78.74 110.49) (width 0.25) (layer "F.Cu") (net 31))
 (segment (start 76.2 118.11) (end 77.47 119.38) (width 0.25) (layer "B.Cu") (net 9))
 (segment (start 77.47 132.08) (end 77.47 119.38) (width 0.25) (layer "B.Cu") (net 9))
 (segment (start 76.2 139.232) (end 76.2 133.35) (width 0.25) (layer "B.Cu") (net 9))
 (segment (start 76.2 115.57) (end 76.2 118.11) (width 0.25) (layer "B.Cu") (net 9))
 (segment (start 76.2 133.35) (end 77.47 132.08) (width 0.25) (layer "B.Cu") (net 9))
 (segment (start 78.74 139.232) (end 78.74 130.81) (width 0.25) (layer "F.Cu") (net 21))
 (segment (start 80.01 132.08) (end 80.01 119.38) (width 0.25) (layer "B.Cu") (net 8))
 (segment (start 78.74 139.232) (end 78.74 133.35) (width 0.25) (layer "B.Cu") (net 8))
 (segment (start 78.74 115.57) (end 78.74 118.11) (width 0.25) (layer "B.Cu") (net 8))
 (segment (start 78.74 118.11) (end 80.01 119.38) (width 0.25) (layer "B.Cu") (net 8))
 (segment (start 78.74 133.35) (end 80.01 132.08) (width 0.25) (layer "B.Cu") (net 8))
 (segment (start 82.55 132.08) (end 81.28 133.35) (width 0.25) (layer "F.Cu") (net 30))
 (segment (start 85.09 125.73) (end 82.55 128.27) (width 0.25) (layer "F.Cu") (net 30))
 (segment (start 82.55 128.27) (end 82.55 132.08) (width 0.25) (layer "F.Cu") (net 30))
 (segment (start 81.28 133.35) (end 81.28 139.232) (width 0.25) (layer "F.Cu") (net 30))
 (segment (start 86.36 111.78) (end 85.09 113.05) (width 0.25) (layer "F.Cu") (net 30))
 (segment (start 85.09 113.05) (end 85.09 125.73) (width 0.25) (layer "F.Cu") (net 30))
 (segment (start 82.55 132.08) (end 82.55 119.38) (width 0.25) (layer "B.Cu") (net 7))
 (segment (start 81.28 139.232) (end 81.28 133.35) (width 0.25) (layer "B.Cu") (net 7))
 (segment (start 81.28 118.11) (end 82.55 119.38) (width 0.25) (layer "B.Cu") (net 7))
 (segment (start 81.28 133.35) (end 82.55 132.08) (width 0.25) (layer "B.Cu") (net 7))
 (segment (start 81.28 115.57) (end 81.28 118.11) (width 0.25) (layer "B.Cu") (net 7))
 (segment (start 83.82 139.192) (end 83.82 130.81) (width 0.25) (layer "F.Cu") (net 23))
 (segment (start 83.82 115.57) (end 83.82 118.11) (width 0.25) (layer "B.Cu") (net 6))
 (segment (start 83.82 118.11) (end 85.09 119.38) (width 0.25) (layer "B.Cu") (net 6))
 (segment (start 85.09 132.08) (end 85.09 119.38) (width 0.25) (layer "B.Cu") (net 6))
 (segment (start 83.82 139.192) (end 83.82 133.35) (width 0.25) (layer "B.Cu") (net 6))
 (segment (start 83.82 133.35) (end 85.09 132.08) (width 0.25) (layer "B.Cu") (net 6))
 (segment (start 86.36 132.08) (end 88.9 134.62) (width 0.25) (layer "F.Cu") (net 24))
 (segment (start 88.9 139.192) (end 88.9 134.62) (width 0.25) (layer "F.Cu") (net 24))
 (segment (start 86.36 130.81) (end 86.36 132.08) (width 0.25) (layer "F.Cu") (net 24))
 (segment (start 88.9 133.35) (end 87.63 132.08) (width 0.25) (layer "B.Cu") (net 5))
 (segment (start 87.63 132.08) (end 87.63 119.38) (width 0.25) (layer "B.Cu") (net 5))
 (segment (start 88.9 139.192) (end 88.9 133.35) (width 0.25) (layer "B.Cu") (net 5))
 (segment (start 86.36 118.11) (end 87.63 119.38) (width 0.25) (layer "B.Cu") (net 5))
 (segment (start 86.36 115.57) (end 86.36 118.11) (width 0.25) (layer "B.Cu") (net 5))
 (segment (start 88.9 130.81) (end 88.9 132.08) (width 0.25) (layer "F.Cu") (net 25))
 (segment (start 88.9 132.08) (end 91.44 134.62) (width 0.25) (layer "F.Cu") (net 25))
 (segment (start 91.44 139.232) (end 91.44 134.62) (width 0.25) (layer "F.Cu") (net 25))
 (segment (start 88.9 115.57) (end 88.9 118.11) (width 0.25) (layer "B.Cu") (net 4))
 (segment (start 90.17 132.08) (end 90.17 119.38) (width 0.25) (layer "B.Cu") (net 4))
 (segment (start 88.9 118.11) (end 90.17 119.38) (width 0.25) (layer "B.Cu") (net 4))
 (segment (start 91.44 133.35) (end 90.17 132.08) (width 0.25) (layer "B.Cu") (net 4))
 (segment (start 91.44 139.232) (end 91.44 133.35) (width 0.25) (layer "B.Cu") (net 4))
 (segment (start 93.98 134.62) (end 91.44 132.08) (width 0.25) (layer "F.Cu") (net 26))
 (segment (start 93.98 139.232) (end 93.98 134.62) (width 0.25) (layer "F.Cu") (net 26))
 (segment (start 91.44 132.08) (end 91.44 130.81) (width 0.25) (layer "F.Cu") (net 26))
 (segment (start 93.98 133.35) (end 92.71 132.08) (width 0.25) (layer "B.Cu") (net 3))
 (segment (start 91.44 118.11) (end 92.71 119.38) (width 0.25) (layer "B.Cu") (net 3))
 (segment (start 93.98 139.232) (end 93.98 133.35) (width 0.25) (layer "B.Cu") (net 3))
 (segment (start 91.44 115.57) (end 91.44 118.11) (width 0.25) (layer "B.Cu") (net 3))
 (segment (start 92.71 132.08) (end 92.71 119.38) (width 0.25) (layer "B.Cu") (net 3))
 (segment (start 96.52 135.89) (end 96.52 139.232) (width 0.25) (layer "F.Cu") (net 29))
 (segment (start 87.63 109.22) (end 87.63 116.84) (width 0.25) (layer "F.Cu") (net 29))
 (segment (start 76.2 111.78) (end 76.2 109.22) (width 0.25) (layer "F.Cu") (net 29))
 (segment (start 76.2 109.22) (end 77.47 107.95) (width 0.25) (layer "F.Cu") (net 29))
 (segment (start 87.63 116.84) (end 92.71 121.92) (width 0.25) (layer "F.Cu") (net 29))
 (segment (start 86.36 107.95) (end 87.63 109.22) (width 0.25) (layer "F.Cu") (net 29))
 (segment (start 92.71 121.92) (end 92.71 132.08) (width 0.25) (layer "F.Cu") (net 29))
 (segment (start 77.47 107.95) (end 86.36 107.95) (width 0.25) (layer "F.Cu") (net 29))
 (segment (start 92.71 132.08) (end 96.52 135.89) (width 0.25) (layer "F.Cu") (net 29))
 (segment (start 96.52 133.35) (end 95.25 132.08) (width 0.25) (layer "B.Cu") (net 2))
 (segment (start 93.98 118.11) (end 95.25 119.38) (width 0.25) (layer "B.Cu") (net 2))
 (segment (start 96.52 139.232) (end 96.52 133.35) (width 0.25) (layer "B.Cu") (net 2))
 (segment (start 95.25 132.08) (end 95.25 119.38) (width 0.25) (layer "B.Cu") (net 2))
 (segment (start 93.98 115.57) (end 93.98 118.11) (width 0.25) (layer "B.Cu") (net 2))
 (segment (start 76.2 130.81) (end 76.2 120.65) (width 0.25) (layer "B.Cu") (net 20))
 (segment (start 74.93 119.38) (end 74.93 113.05) (width 0.25) (layer "B.Cu") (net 20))
 (segment (start 76.2 120.65) (end 74.93 119.38) (width 0.25) (layer "B.Cu") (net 20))
 (segment (start 74.93 113.05) (end 73.66 111.78) (width 0.25) (layer "B.Cu") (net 20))
 (segment (start 81.28 128.27) (end 81.28 130.81) (width 0.25) (layer "F.Cu") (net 22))
 (segment (start 80.155 127.145) (end 81.28 128.27) (width 0.25) (layer "F.Cu") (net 22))
 (segment (start 81.28 111.78) (end 80.155 112.905) (width 0.25) (layer "F.Cu") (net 22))
 (segment (start 80.155 112.905) (end 80.155 127.145) (width 0.25) (layer "F.Cu") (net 22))
 (segment (start 86.039009 104.16) (end 86.36 104.16) (width 0.25) (layer "F.Cu") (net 33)))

